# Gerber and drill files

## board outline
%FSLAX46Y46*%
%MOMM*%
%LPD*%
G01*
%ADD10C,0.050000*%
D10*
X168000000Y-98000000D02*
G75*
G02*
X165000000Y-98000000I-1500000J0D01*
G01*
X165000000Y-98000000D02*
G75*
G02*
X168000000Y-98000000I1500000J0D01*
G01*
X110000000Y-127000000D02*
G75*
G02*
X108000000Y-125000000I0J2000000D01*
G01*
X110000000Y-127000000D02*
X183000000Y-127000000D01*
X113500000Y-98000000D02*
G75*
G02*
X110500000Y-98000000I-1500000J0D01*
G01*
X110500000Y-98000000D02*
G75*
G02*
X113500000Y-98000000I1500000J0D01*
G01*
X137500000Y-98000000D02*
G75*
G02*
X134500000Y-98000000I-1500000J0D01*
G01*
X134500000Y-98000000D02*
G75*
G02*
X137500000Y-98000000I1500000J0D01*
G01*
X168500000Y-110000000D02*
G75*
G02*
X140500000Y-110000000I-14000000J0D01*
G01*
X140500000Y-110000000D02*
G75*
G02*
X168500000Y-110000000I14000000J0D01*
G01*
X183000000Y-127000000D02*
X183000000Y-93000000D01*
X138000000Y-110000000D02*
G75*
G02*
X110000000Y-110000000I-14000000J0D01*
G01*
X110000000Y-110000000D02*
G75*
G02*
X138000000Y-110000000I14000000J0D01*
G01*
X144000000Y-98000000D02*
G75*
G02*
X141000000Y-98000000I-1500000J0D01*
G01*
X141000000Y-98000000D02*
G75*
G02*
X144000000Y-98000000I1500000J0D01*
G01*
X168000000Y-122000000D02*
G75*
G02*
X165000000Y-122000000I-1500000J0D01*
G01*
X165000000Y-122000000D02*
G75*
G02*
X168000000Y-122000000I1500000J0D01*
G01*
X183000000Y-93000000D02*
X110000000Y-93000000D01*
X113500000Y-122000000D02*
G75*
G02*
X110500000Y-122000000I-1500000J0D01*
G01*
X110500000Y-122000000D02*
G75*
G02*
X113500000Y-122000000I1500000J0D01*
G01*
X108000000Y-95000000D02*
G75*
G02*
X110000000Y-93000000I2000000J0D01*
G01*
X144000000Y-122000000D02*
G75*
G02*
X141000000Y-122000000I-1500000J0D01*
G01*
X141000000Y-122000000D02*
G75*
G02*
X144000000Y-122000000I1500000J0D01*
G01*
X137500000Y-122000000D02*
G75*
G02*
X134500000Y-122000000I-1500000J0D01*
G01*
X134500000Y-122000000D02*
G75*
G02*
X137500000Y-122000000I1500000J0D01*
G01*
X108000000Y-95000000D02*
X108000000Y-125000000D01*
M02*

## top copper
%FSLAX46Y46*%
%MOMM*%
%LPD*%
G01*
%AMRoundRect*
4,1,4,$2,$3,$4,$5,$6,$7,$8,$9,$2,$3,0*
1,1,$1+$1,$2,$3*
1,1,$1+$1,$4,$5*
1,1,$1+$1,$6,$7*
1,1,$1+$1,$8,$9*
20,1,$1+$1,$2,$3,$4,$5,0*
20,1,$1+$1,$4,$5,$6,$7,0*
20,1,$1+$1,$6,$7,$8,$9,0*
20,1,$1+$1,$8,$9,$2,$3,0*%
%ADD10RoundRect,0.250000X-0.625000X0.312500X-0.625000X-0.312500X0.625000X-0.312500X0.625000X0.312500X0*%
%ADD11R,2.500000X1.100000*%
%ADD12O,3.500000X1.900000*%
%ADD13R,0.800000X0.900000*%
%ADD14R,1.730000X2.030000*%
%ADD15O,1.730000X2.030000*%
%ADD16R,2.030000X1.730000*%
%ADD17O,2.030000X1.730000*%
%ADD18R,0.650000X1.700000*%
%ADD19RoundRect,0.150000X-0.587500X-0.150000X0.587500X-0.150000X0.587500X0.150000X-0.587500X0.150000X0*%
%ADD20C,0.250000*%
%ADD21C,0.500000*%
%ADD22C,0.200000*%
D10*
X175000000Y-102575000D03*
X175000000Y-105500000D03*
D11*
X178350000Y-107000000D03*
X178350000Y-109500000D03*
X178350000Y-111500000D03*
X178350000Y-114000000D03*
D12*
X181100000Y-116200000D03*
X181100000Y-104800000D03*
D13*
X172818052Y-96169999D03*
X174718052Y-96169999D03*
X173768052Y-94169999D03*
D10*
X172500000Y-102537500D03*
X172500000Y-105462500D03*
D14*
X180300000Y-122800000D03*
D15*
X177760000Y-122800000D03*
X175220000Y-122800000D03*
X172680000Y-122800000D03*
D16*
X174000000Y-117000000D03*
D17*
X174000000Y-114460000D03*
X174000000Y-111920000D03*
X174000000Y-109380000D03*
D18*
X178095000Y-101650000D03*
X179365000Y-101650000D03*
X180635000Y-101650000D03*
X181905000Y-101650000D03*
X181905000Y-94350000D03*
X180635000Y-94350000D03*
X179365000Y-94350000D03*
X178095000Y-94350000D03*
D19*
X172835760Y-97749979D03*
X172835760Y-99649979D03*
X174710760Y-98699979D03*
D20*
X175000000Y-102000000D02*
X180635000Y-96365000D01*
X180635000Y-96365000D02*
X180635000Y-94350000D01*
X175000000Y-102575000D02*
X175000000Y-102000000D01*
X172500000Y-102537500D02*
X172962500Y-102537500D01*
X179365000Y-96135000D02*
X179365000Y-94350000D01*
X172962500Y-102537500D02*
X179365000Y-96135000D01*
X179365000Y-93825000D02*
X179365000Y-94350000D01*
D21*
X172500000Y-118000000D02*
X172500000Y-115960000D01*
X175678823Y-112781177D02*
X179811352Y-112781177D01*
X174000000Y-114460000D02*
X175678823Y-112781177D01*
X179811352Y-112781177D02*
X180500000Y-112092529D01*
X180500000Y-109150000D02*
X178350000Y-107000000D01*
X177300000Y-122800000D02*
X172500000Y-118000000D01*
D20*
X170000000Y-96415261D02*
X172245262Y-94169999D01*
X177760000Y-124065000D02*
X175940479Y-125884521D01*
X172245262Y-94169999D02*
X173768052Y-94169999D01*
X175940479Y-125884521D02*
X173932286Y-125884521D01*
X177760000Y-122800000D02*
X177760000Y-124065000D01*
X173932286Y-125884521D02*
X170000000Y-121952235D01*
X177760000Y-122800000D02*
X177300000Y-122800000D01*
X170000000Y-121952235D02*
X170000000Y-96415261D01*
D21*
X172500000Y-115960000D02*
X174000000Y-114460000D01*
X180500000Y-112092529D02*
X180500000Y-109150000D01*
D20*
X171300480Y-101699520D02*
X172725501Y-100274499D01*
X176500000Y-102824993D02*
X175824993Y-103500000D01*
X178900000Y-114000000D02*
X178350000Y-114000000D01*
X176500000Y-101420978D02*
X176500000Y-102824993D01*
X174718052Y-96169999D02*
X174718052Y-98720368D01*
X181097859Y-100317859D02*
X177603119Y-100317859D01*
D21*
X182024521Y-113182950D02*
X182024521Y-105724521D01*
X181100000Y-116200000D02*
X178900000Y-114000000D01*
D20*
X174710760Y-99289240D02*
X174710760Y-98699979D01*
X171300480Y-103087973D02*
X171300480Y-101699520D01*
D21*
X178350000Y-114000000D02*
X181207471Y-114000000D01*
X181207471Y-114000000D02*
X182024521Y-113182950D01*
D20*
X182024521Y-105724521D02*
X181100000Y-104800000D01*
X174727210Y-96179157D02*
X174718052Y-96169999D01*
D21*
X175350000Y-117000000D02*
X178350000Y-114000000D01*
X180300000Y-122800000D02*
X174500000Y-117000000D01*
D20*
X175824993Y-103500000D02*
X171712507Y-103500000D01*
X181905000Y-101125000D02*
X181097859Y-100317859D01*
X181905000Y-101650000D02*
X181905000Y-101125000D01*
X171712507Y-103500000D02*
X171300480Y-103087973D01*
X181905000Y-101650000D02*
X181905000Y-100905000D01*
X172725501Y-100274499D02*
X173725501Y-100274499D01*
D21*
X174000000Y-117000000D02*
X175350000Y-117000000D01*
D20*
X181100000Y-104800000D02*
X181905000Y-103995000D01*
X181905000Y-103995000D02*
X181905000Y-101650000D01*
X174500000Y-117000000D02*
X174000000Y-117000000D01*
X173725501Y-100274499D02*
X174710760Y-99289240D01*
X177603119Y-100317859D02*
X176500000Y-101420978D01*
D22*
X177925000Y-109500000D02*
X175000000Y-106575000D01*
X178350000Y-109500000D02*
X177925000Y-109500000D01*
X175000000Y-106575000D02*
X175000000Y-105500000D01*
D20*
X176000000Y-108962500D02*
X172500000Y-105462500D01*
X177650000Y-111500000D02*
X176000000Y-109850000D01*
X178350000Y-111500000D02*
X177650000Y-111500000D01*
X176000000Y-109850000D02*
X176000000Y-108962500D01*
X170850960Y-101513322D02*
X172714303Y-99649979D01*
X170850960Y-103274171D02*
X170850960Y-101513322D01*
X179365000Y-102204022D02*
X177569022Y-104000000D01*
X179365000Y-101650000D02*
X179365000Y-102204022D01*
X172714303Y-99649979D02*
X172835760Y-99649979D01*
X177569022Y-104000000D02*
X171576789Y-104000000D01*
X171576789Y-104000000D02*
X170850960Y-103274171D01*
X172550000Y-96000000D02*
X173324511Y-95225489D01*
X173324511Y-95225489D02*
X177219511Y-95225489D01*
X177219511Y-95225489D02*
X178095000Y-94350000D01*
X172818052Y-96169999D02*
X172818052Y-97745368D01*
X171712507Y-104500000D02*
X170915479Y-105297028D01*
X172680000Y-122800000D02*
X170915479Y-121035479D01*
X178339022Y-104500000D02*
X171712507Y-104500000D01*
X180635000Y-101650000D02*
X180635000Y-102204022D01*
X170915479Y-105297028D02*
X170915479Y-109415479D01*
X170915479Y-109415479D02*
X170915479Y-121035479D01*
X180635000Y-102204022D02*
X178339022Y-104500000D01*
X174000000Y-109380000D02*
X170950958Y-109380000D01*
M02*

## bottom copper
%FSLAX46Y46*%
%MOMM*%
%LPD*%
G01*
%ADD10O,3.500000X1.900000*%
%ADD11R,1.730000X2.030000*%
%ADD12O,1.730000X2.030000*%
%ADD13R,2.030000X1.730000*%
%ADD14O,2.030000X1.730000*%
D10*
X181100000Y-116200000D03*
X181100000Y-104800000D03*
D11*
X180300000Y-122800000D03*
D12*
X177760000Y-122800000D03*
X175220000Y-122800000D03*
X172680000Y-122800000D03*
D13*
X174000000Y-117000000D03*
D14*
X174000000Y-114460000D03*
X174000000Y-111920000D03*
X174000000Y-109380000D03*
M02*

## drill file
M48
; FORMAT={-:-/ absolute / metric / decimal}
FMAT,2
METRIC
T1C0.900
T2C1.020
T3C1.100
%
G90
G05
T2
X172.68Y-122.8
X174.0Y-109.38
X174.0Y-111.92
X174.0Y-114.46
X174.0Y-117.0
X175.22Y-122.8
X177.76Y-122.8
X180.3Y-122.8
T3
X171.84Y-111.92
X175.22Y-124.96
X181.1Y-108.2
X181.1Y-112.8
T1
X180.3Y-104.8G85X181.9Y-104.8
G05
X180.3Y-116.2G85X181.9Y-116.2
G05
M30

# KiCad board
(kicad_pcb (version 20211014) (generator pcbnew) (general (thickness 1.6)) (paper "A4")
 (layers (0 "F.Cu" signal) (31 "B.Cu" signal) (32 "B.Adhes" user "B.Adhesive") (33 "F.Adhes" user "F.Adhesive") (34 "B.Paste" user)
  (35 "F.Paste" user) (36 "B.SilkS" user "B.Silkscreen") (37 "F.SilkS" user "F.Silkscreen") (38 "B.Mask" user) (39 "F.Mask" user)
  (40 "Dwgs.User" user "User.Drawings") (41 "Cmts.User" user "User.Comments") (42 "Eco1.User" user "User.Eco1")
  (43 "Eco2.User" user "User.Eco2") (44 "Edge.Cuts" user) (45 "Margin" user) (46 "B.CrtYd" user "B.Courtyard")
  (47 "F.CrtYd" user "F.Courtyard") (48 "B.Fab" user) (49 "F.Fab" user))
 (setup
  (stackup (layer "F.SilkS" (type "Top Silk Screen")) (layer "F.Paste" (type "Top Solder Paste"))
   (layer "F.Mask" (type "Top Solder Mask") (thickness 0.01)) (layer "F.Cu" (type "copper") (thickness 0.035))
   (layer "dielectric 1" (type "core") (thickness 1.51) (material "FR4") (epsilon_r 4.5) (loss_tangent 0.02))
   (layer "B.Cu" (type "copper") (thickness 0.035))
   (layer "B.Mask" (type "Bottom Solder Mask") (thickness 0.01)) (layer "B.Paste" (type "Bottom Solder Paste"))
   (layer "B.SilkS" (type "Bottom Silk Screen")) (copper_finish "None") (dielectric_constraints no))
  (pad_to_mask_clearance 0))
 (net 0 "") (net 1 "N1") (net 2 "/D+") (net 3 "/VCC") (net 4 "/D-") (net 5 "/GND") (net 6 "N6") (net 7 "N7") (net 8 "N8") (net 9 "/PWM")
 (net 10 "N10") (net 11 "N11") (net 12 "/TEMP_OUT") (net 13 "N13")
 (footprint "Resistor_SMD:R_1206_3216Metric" (layer "F.Cu") (at 175 104.0375 -90)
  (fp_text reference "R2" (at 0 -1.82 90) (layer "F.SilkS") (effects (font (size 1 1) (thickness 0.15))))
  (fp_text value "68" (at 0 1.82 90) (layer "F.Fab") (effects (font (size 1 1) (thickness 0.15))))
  (pad "1" smd roundrect locked (at -1.4625 0 270) (size 1.125 1.75) (layers "F.Cu" "F.Paste" "F.Mask") (roundrect_rratio 0.222222)
   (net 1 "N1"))
  (pad "2" smd roundrect locked (at 1.4625 0 270) (size 1.125 1.75) (layers "F.Cu" "F.Paste" "F.Mask") (roundrect_rratio 0.222222)
   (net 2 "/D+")))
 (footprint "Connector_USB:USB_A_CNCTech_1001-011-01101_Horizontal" (layer "F.Cu") (at 188 110.5)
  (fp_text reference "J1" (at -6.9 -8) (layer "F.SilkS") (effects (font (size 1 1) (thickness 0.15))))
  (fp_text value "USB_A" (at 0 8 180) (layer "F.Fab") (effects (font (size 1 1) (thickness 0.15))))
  (pad "" np_thru_hole circle (at -6.9 -2.3) (size 1.1 1.1) (drill 1.1) (layers *.Cu *.Mask))
  (pad "" np_thru_hole circle (at -6.9 2.3) (size 1.1 1.1) (drill 1.1) (layers *.Cu *.Mask))
  (pad "1" smd rect (at -9.65 -3.5) (size 2.5 1.1) (layers "F.Cu" "F.Paste" "F.Mask") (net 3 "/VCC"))
  (pad "2" smd rect (at -9.65 -1) (size 2.5 1.1) (layers "F.Cu" "F.Paste" "F.Mask") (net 2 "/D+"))
  (pad "3" smd rect (at -9.65 1) (size 2.5 1.1) (layers "F.Cu" "F.Paste" "F.Mask") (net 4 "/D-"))
  (pad "4" smd rect (at -9.65 3.5) (size 2.5 1.1) (layers "F.Cu" "F.Paste" "F.Mask") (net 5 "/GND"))
  (pad "5" thru_hole oval (at -6.9 5.7) (size 3.5 1.9) (drill oval 2.5 0.9) (layers *.Cu *.Mask) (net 5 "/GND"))
  (pad "5" thru_hole oval (at -6.9 -5.7) (size 3.5 1.9) (drill oval 2.5 0.9) (layers *.Cu *.Mask) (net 5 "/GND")))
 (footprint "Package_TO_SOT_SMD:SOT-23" (layer "F.Cu") (at 173.768052 95.169999 90)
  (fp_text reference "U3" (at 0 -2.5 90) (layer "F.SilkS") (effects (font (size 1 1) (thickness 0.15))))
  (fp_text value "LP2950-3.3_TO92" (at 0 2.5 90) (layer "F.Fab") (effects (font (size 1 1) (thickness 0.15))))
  (pad "1" smd rect locked (at -1 -0.95 90) (size 0.9 0.8) (layers "F.Cu" "F.Paste" "F.Mask") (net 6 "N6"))
  (pad "2" smd rect locked (at -1 0.95 90) (size 0.9 0.8) (layers "F.Cu" "F.Paste" "F.Mask") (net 5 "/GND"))
  (pad "3" smd rect locked (at 1 0 90) (size 0.9 0.8) (layers "F.Cu" "F.Paste" "F.Mask") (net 3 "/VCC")))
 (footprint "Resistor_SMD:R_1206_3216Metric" (layer "F.Cu") (at 172.5 104 -90)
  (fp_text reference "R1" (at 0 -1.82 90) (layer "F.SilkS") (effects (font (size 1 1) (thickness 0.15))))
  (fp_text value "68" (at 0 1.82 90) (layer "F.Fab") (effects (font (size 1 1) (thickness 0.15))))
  (pad "1" smd roundrect locked (at -1.4625 0 270) (size 1.125 1.75) (layers "F.Cu" "F.Paste" "F.Mask") (roundrect_rratio 0.222222)
   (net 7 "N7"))
  (pad "2" smd roundrect locked (at 1.4625 0 270) (size 1.125 1.75) (layers "F.Cu" "F.Paste" "F.Mask") (roundrect_rratio 0.222222)
   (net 4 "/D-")))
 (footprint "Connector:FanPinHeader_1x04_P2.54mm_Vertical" (layer "F.Cu") (at 180.3 122.8 180)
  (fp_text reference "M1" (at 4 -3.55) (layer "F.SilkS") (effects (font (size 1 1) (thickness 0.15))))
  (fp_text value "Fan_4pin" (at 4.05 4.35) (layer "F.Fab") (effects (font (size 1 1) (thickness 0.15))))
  (pad "" np_thru_hole circle locked (at 5.08 -2.16 270) (size 1.1 1.1) (drill 1.1) (layers *.Cu *.Mask))
  (pad "1" thru_hole rect locked (at 0 0 270) (size 2.03 1.73) (drill 1.02) (layers *.Cu *.Mask) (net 5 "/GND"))
  (pad "2" thru_hole oval locked (at 2.54 0 270) (size 2.03 1.73) (drill 1.02) (layers *.Cu *.Mask) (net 3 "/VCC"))
  (pad "3" thru_hole oval locked (at 5.08 0 270) (size 2.03 1.73) (drill 1.02) (layers *.Cu *.Mask) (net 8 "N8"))
  (pad "4" thru_hole oval locked (at 7.62 0 270) (size 2.03 1.73) (drill 1.02) (layers *.Cu *.Mask) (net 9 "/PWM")))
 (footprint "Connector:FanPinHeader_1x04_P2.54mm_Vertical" (layer "F.Cu") (at 174 117 90)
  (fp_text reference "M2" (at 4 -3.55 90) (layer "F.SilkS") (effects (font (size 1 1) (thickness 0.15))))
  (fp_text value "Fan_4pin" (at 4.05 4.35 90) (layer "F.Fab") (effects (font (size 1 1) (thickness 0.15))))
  (pad "" np_thru_hole circle locked (at 5.08 -2.16 180) (size 1.1 1.1) (drill 1.1) (layers *.Cu *.Mask))
  (pad "1" thru_hole rect locked (at 0 0 180) (size 2.03 1.73) (drill 1.02) (layers *.Cu *.Mask) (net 5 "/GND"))
  (pad "2" thru_hole oval locked (at 2.54 0 180) (size 2.03 1.73) (drill 1.02) (layers *.Cu *.Mask) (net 3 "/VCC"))
  (pad "3" thru_hole oval locked (at 5.08 0 180) (size 2.03 1.73) (drill 1.02) (layers *.Cu *.Mask) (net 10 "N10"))
  (pad "4" thru_hole oval locked (at 7.62 0 180) (size 2.03 1.73) (drill 1.02) (layers *.Cu *.Mask) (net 9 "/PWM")))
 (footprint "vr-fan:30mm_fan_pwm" (layer "F.Cu") (at 124 110)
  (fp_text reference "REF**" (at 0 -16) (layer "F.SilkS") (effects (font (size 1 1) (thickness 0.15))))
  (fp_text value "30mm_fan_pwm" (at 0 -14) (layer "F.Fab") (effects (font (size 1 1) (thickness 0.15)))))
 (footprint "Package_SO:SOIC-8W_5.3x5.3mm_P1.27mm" (layer "F.Cu") (at 180 98 90)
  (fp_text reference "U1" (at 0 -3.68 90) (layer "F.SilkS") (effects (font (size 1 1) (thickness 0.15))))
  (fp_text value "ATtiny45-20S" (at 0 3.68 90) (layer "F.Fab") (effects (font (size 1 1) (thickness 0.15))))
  (pad "1" smd rect (at -3.65 -1.905 90) (size 1.7 0.65) (layers "F.Cu" "F.Paste" "F.Mask") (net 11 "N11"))
  (pad "2" smd rect (at -3.65 -0.635 90) (size 1.7 0.65) (layers "F.Cu" "F.Paste" "F.Mask") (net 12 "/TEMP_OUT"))
  (pad "3" smd rect (at -3.65 0.635 90) (size 1.7 0.65) (layers "F.Cu" "F.Paste" "F.Mask") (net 9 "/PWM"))
  (pad "4" smd rect (at -3.65 1.905 90) (size 1.7 0.65) (layers "F.Cu" "F.Paste" "F.Mask") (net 5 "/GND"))
  (pad "5" smd rect (at 3.65 1.905 90) (size 1.7 0.65) (layers "F.Cu" "F.Paste" "F.Mask") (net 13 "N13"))
  (pad "6" smd rect (at 3.65 0.635 90) (size 1.7 0.65) (layers "F.Cu" "F.Paste" "F.Mask") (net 1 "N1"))
  (pad "7" smd rect (at 3.65 -0.635 90) (size 1.7 0.65) (layers "F.Cu" "F.Paste" "F.Mask") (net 7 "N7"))
  (pad "8" smd rect (at 3.65 -1.905 90) (size 1.7 0.65) (layers "F.Cu" "F.Paste" "F.Mask") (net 6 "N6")))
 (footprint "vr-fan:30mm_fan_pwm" (layer "F.Cu") (at 154.5 110)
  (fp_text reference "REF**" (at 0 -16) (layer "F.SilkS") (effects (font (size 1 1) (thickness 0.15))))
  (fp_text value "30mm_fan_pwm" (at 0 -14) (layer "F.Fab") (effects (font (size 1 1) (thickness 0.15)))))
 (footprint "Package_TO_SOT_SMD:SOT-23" (layer "F.Cu") (at 173.77326 98.699979)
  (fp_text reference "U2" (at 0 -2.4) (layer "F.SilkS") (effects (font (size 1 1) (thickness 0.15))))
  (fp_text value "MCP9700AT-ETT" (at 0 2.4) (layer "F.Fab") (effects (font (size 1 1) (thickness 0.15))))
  (pad "1" smd roundrect (at -0.9375 -0.95) (size 1.475 0.6) (layers "F.Cu" "F.Paste" "F.Mask") (roundrect_rratio 0.25) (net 6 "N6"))
  (pad "2" smd roundrect (at -0.9375 0.95) (size 1.475 0.6) (layers "F.Cu" "F.Paste" "F.Mask") (roundrect_rratio 0.25) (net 12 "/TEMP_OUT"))
  (pad "3" smd roundrect (at 0.9375 0) (size 1.475 0.6) (layers "F.Cu" "F.Paste" "F.Mask") (roundrect_rratio 0.25) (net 5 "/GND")))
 (gr_circle (center 166.5 98) (end 166.5 99.5) (layer "Edge.Cuts") (width 0.05) (fill none))
 (gr_arc (start 110 127) (mid 108.585786 126.414214) (end 108 125) (layer "Edge.Cuts") (width 0.05))
 (gr_line (start 110 127) (end 183 127) (layer "Edge.Cuts") (width 0.05))
 (gr_circle (center 112 98) (end 112 99.5) (layer "Edge.Cuts") (width 0.05) (fill none))
 (gr_circle (center 136 98) (end 136 99.5) (layer "Edge.Cuts") (width 0.05) (fill none))
 (gr_circle (center 154.5 110) (end 154.5 124) (layer "Edge.Cuts") (width 0.05) (fill none))
 (gr_line (start 183 127) (end 183 93) (layer "Edge.Cuts") (width 0.05))
 (gr_circle (center 124 110) (end 124 124) (layer "Edge.Cuts") (width 0.05) (fill none))
 (gr_circle (center 142.5 98) (end 142.5 99.5) (layer "Edge.Cuts") (width 0.05) (fill none))
 (gr_circle (center 166.5 122) (end 166.5 123.5) (layer "Edge.Cuts") (width 0.05) (fill none))
 (gr_line (start 183 93) (end 110 93) (layer "Edge.Cuts") (width 0.05))
 (gr_circle (center 112 122) (end 112 123.5) (layer "Edge.Cuts") (width 0.05) (fill none))
 (gr_arc (start 108 95) (mid 108.585786 93.585786) (end 110 93) (layer "Edge.Cuts") (width 0.05))
 (gr_circle (center 142.5 122) (end 142.5 123.5) (layer "Edge.Cuts") (width 0.05) (fill none))
 (gr_circle (center 136 122) (end 136 123.5) (layer "Edge.Cuts") (width 0.05) (fill none))
 (gr_line (start 108 95) (end 108 125) (layer "Edge.Cuts") (width 0.05))
 (segment (start 175 102) (end 180.635 96.365) (width 0.25) (layer "F.Cu") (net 1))
 (segment (start 180.635 96.365) (end 180.635 94.35) (width 0.25) (layer "F.Cu") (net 1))
 (segment (start 175 102.575) (end 175 102) (width 0.25) (layer "F.Cu") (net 1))
 (segment (start 172.5 102.5375) (end 172.9625 102.5375) (width 0.25) (layer "F.Cu") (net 7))
 (segment (start 179.365 96.135) (end 179.365 94.35) (width 0.25) (layer "F.Cu") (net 7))
 (segment (start 172.9625 102.5375) (end 179.365 96.135) (width 0.25) (layer "F.Cu") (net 7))
 (segment (start 179.365 93.825) (end 179.365 94.35) (width 0.25) (layer "F.Cu") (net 7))
 (segment (start 172.5 118) (end 172.5 115.96) (width 0.5) (layer "F.Cu") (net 3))
 (segment (start 175.678823 112.781177) (end 179.811352 112.781177) (width 0.5) (layer "F.Cu") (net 3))
 (segment (start 174 114.46) (end 175.678823 112.781177) (width 0.5) (layer "F.Cu") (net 3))
 (segment (start 179.811352 112.781177) (end 180.5 112.092529) (width 0.5) (layer "F.Cu") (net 3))
 (segment (start 180.5 109.15) (end 178.35 107) (width 0.5) (layer "F.Cu") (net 3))
 (segment (start 177.3 122.8) (end 172.5 118) (width 0.5) (layer "F.Cu") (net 3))
 (segment (start 170 96.415261) (end 172.245262 94.169999) (width 0.25) (layer "F.Cu") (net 3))
 (segment (start 177.76 124.065) (end 175.940479 125.884521) (width 0.25) (layer "F.Cu") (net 3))
 (segment (start 172.245262 94.169999) (end 173.768052 94.169999) (width 0.25) (layer "F.Cu") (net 3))
 (segment (start 175.940479 125.884521) (end 173.932286 125.884521) (width 0.25) (layer "F.Cu") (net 3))
 (segment (start 177.76 122.8) (end 177.76 124.065) (width 0.25) (layer "F.Cu") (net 3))
 (segment (start 173.932286 125.884521) (end 170 121.952235) (width 0.25) (layer "F.Cu") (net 3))
 (segment (start 177.76 122.8) (end 177.3 122.8) (width 0.25) (layer "F.Cu") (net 3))
 (segment (start 170 121.952235) (end 170 96.415261) (width 0.25) (layer "F.Cu") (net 3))
 (segment (start 172.5 115.96) (end 174 114.46) (width 0.5) (layer "F.Cu") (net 3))
 (segment (start 180.5 112.092529) (end 180.5 109.15) (width 0.5) (layer "F.Cu") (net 3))
 (segment (start 171.30048 101.69952) (end 172.725501 100.274499) (width 0.25) (layer "F.Cu") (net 5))
 (segment (start 176.5 102.824993) (end 175.824993 103.5) (width 0.25) (layer "F.Cu") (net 5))
 (segment (start 178.9 114) (end 178.35 114) (width 0.25) (layer "F.Cu") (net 5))
 (segment (start 176.5 101.420978) (end 176.5 102.824993) (width 0.25) (layer "F.Cu") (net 5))
 (segment (start 174.718052 96.169999) (end 174.718052 98.720368) (width 0.25) (layer "F.Cu") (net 5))
 (segment (start 181.097859 100.317859) (end 177.603119 100.317859) (width 0.25) (layer "F.Cu") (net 5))
 (segment (start 182.024521 113.18295) (end 182.024521 105.724521) (width 0.5) (layer "F.Cu") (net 5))
 (segment (start 181.1 116.2) (end 178.9 114) (width 0.5) (layer "F.Cu") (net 5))
 (segment (start 174.71076 99.28924) (end 174.71076 98.699979) (width 0.25) (layer "F.Cu") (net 5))
 (segment (start 171.30048 103.087973) (end 171.30048 101.69952) (width 0.25) (layer "F.Cu") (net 5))
 (segment (start 178.35 114) (end 181.207471 114) (width 0.5) (layer "F.Cu") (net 5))
 (segment (start 181.207471 114) (end 182.024521 113.18295) (width 0.5) (layer "F.Cu") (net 5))
 (segment (start 182.024521 105.724521) (end 181.1 104.8) (width 0.25) (layer "F.Cu") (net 5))
 (segment (start 174.72721 96.179157) (end 174.718052 96.169999) (width 0.25) (layer "F.Cu") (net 5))
 (segment (start 175.35 117) (end 178.35 114) (width 0.5) (layer "F.Cu") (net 5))
 (segment (start 180.3 122.8) (end 174.5 117) (width 0.5) (layer "F.Cu") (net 5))
 (segment (start 175.824993 103.5) (end 171.712507 103.5) (width 0.25) (layer "F.Cu") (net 5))
 (segment (start 181.905 101.125) (end 181.097859 100.317859) (width 0.25) (layer "F.Cu") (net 5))
 (segment (start 181.905 101.65) (end 181.905 101.125) (width 0.25) (layer "F.Cu") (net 5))
 (segment (start 171.712507 103.5) (end 171.30048 103.087973) (width 0.25) (layer "F.Cu") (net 5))
 (segment (start 181.905 101.65) (end 181.905 100.905) (width 0.25) (layer "F.Cu") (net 5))
 (segment (start 172.725501 100.274499) (end 173.725501 100.274499) (width 0.25) (layer "F.Cu") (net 5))
 (segment (start 174 117) (end 175.35 117) (width 0.5) (layer "F.Cu") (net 5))
 (segment (start 181.1 104.8) (end 181.905 103.995) (width 0.25) (layer "F.Cu") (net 5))
 (segment (start 181.905 103.995) (end 181.905 101.65) (width 0.25) (layer "F.Cu") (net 5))
 (segment (start 174.5 117) (end 174 117) (width 0.25) (layer "F.Cu") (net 5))
 (segment (start 173.725501 100.274499) (end 174.71076 99.28924) (width 0.25) (layer "F.Cu") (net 5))
 (segment (start 177.603119 100.317859) (end 176.5 101.420978) (width 0.25) (layer "F.Cu") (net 5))
 (segment (start 177.925 109.5) (end 175 106.575) (width 0.2) (layer "F.Cu") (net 2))
 (segment (start 178.35 109.5) (end 177.925 109.5) (width 0.2) (layer "F.Cu") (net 2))
 (segment (start 175 106.575) (end 175 105.5) (width 0.2) (layer "F.Cu") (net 2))
 (segment (start 176 108.9625) (end 172.5 105.4625) (width 0.25) (layer "F.Cu") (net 4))
 (segment (start 177.65 111.5) (end 176 109.85) (width 0.25) (layer "F.Cu") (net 4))
 (segment (start 178.35 111.5) (end 177.65 111.5) (width 0.25) (layer "F.Cu") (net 4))
 (segment (start 176 109.85) (end 176 108.9625) (width 0.25) (layer "F.Cu") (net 4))
 (segment (start 170.85096 101.513322) (end 172.714303 99.649979) (width 0.25) (layer "F.Cu") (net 12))
 (segment (start 170.85096 103.274171) (end 170.85096 101.513322) (width 0.25) (layer "F.Cu") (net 12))
 (segment (start 179.365 102.204022) (end 177.569022 104) (width 0.25) (layer "F.Cu") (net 12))
 (segment (start 179.365 101.65) (end 179.365 102.204022) (width 0.25) (layer "F.Cu") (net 12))
 (segment (start 172.714303 99.649979) (end 172.83576 99.649979) (width 0.25) (layer "F.Cu") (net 12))
 (segment (start 177.569022 104) (end 171.576789 104) (width 0.25) (layer "F.Cu") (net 12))
 (segment (start 171.576789 104) (end 170.85096 103.274171) (width 0.25) (layer "F.Cu") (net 12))
 (segment (start 172.55 96) (end 173.324511 95.225489) (width 0.25) (layer "F.Cu") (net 6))
 (segment (start 173.324511 95.225489) (end 177.219511 95.225489) (width 0.25) (layer "F.Cu") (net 6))
 (segment (start 177.219511 95.225489) (end 178.095 94.35) (width 0.25) (layer "F.Cu") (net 6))
 (segment (start 172.818052 96.169999) (end 172.818052 97.745368) (width 0.25) (layer "F.Cu") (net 6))
 (segment (start 171.712507 104.5) (end 170.915479 105.297028) (width 0.25) (layer "F.Cu") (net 9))
 (segment (start 172.68 122.8) (end 170.915479 121.035479) (width 0.25) (layer "F.Cu") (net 9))
 (segment (start 178.339022 104.5) (end 171.712507 104.5) (width 0.25) (layer "F.Cu") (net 9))
 (segment (start 180.635 101.65) (end 180.635 102.204022) (width 0.25) (layer "F.Cu") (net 9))
 (segment (start 170.915479 105.297028) (end 170.915479 109.415479) (width 0.25) (layer "F.Cu") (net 9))
 (segment (start 170.915479 109.415479) (end 170.915479 121.035479) (width 0.25) (layer "F.Cu") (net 9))
 (segment (start 180.635 102.204022) (end 178.339022 104.5) (width 0.25) (layer "F.Cu") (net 9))
 (segment (start 174 109.38) (end 170.950958 109.38) (width 0.25) (layer "F.Cu") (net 9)))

